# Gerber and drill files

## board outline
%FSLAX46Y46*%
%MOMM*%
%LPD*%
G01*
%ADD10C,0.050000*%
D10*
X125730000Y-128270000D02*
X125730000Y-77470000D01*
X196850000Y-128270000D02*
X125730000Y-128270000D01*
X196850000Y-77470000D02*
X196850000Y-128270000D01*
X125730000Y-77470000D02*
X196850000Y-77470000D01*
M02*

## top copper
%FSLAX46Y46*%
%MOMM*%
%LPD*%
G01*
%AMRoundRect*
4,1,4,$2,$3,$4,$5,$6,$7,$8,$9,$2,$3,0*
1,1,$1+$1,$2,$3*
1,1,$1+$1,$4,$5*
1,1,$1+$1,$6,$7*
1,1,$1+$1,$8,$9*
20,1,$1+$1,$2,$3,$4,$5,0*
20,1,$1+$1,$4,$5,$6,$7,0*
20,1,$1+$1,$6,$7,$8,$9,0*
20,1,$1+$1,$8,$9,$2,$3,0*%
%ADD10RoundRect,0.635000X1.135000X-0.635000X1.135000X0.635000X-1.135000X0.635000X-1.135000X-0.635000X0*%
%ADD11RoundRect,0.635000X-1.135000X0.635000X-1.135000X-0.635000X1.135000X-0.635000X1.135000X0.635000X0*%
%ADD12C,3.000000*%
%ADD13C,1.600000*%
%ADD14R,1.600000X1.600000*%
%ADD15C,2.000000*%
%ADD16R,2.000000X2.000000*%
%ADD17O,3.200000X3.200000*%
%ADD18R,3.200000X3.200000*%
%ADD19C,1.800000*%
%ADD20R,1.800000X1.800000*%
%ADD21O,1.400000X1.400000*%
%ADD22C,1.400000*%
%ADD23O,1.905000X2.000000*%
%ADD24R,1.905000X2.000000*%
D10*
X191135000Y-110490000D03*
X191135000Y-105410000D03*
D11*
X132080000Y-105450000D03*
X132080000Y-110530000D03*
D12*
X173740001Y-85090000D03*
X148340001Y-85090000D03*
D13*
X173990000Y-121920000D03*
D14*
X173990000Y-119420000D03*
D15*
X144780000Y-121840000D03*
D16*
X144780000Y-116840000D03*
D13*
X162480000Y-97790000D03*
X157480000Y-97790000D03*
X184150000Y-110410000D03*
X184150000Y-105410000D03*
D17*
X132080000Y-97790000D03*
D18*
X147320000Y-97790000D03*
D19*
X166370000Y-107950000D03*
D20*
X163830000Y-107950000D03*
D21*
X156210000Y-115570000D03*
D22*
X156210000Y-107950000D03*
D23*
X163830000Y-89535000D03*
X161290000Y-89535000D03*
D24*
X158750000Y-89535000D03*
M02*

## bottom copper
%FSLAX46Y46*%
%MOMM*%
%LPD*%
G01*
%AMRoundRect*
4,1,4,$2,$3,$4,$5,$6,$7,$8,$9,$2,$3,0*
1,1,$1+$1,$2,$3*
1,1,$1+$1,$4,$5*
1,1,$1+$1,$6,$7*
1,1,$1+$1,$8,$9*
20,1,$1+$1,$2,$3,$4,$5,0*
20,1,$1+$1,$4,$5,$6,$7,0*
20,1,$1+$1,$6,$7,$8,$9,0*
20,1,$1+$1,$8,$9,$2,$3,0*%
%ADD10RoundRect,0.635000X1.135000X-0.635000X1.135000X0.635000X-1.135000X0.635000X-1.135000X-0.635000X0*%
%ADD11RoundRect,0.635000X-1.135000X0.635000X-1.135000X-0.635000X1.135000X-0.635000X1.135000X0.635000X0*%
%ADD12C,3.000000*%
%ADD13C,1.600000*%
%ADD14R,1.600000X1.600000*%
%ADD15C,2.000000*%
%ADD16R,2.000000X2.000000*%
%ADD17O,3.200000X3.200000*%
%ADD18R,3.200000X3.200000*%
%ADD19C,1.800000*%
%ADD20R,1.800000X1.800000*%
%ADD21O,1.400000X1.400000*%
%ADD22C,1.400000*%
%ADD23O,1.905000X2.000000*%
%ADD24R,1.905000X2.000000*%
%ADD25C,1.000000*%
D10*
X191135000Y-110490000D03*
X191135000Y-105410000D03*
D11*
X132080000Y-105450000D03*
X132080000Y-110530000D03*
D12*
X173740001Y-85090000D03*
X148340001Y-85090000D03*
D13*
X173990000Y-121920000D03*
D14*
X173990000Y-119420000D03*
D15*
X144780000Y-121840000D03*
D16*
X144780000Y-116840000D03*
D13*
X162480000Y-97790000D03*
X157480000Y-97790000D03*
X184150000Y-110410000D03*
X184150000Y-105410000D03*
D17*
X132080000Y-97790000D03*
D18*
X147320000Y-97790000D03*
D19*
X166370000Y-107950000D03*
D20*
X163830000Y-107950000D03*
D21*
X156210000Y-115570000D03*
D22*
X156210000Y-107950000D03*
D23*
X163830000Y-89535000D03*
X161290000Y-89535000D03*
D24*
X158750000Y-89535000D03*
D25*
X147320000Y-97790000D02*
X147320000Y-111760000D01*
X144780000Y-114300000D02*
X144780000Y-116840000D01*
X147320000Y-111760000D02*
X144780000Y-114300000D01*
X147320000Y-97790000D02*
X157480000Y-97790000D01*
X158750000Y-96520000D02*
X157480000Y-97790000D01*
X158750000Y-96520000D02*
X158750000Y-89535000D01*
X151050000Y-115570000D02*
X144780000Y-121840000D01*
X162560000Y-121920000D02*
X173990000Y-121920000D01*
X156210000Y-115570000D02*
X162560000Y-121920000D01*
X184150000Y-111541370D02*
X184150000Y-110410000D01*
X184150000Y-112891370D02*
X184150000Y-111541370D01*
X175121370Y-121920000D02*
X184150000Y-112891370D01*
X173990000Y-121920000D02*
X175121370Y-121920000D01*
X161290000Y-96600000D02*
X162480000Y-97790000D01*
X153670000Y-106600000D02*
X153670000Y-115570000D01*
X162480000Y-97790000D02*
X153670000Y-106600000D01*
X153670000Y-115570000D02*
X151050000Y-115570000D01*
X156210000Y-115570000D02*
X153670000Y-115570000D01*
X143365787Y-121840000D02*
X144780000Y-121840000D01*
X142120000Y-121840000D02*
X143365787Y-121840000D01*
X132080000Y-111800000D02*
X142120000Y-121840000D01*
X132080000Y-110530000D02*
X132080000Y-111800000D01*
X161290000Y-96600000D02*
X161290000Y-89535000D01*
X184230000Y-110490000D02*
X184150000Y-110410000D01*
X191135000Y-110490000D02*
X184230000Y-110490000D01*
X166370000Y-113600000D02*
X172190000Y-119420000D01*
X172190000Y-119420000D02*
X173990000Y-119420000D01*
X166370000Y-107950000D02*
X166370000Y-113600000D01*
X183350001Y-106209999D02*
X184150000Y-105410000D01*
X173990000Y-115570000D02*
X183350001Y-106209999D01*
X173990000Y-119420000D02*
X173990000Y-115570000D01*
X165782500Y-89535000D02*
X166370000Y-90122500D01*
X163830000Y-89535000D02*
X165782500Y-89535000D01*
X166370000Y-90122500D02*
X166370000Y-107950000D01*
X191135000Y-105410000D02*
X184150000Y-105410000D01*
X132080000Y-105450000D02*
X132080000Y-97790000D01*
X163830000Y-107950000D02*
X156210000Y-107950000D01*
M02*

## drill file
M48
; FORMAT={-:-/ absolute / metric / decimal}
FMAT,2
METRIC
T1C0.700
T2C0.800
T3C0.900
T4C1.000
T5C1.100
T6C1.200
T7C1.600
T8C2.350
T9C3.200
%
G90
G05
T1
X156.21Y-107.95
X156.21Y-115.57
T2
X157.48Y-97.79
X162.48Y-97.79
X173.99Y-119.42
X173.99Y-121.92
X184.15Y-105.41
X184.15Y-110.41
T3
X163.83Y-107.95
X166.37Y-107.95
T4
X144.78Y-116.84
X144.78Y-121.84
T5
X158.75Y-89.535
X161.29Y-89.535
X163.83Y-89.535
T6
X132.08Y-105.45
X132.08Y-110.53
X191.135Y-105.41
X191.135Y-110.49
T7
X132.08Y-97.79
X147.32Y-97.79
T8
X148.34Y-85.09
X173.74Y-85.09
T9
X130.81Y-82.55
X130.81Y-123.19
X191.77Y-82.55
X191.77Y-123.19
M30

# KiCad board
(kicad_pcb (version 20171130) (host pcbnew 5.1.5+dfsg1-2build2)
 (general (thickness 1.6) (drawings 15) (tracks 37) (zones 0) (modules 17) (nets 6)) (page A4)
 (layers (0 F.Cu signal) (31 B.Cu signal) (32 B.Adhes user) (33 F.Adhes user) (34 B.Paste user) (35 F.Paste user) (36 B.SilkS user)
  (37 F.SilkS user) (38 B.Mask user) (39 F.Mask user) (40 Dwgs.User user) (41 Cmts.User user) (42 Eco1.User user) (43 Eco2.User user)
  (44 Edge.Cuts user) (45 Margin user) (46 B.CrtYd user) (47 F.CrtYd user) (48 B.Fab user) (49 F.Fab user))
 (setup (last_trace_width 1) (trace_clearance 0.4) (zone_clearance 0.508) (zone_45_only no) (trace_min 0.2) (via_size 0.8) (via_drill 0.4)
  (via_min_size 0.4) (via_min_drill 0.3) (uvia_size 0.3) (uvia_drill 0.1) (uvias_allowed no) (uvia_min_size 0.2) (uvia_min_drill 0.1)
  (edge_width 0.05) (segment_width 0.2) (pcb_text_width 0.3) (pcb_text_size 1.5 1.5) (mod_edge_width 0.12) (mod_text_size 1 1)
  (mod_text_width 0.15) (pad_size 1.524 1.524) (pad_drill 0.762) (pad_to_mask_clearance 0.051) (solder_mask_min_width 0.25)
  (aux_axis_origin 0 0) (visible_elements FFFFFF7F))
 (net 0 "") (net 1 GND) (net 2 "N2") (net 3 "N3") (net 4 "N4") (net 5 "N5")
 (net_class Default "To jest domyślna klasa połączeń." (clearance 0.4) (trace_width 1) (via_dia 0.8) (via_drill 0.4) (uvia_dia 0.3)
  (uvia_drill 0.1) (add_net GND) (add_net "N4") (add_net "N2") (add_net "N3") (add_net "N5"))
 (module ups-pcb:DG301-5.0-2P (layer F.Cu) (at 191.135 107.99 90)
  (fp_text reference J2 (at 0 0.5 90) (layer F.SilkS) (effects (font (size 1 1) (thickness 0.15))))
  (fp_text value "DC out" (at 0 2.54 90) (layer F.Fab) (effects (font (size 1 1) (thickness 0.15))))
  (pad 1 thru_hole roundrect (at -2.5 0 90) (size 2.54 3.54) (drill 1.2) (layers *.Cu *.Mask) (roundrect_rratio 0.25) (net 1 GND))
  (pad 2 thru_hole roundrect (at 2.58 0 90) (size 2.54 3.54) (drill 1.2) (layers *.Cu *.Mask) (roundrect_rratio 0.25) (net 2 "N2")))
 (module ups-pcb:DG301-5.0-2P (layer F.Cu) (at 132.08 107.95 270)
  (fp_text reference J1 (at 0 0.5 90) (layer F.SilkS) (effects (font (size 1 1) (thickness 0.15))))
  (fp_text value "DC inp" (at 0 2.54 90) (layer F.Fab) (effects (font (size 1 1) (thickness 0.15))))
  (pad 1 thru_hole roundrect (at -2.5 0 270) (size 2.54 3.54) (drill 1.2) (layers *.Cu *.Mask) (roundrect_rratio 0.25) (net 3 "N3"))
  (pad 2 thru_hole roundrect (at 2.58 0 270) (size 2.54 3.54) (drill 1.2) (layers *.Cu *.Mask) (roundrect_rratio 0.25) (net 1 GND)))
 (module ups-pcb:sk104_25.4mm (layer F.Cu) (at 161.040001 85.09)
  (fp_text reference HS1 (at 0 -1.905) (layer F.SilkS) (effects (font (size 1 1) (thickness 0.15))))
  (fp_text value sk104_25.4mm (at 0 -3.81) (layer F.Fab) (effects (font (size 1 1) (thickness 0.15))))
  (pad "" np_thru_hole circle (at 12.7 0) (size 3 3) (drill 2.35) (layers *.Cu *.Mask))
  (pad "" np_thru_hole circle (at -12.7 0) (size 3 3) (drill 2.35) (layers *.Cu *.Mask)))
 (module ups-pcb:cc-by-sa (layer F.Cu) (at 159.385 121.92)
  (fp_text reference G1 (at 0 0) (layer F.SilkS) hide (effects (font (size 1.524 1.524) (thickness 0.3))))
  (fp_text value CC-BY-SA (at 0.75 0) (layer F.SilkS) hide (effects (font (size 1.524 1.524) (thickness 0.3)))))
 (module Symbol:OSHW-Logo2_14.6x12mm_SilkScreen (layer F.Cu) (at 186.055 93.98)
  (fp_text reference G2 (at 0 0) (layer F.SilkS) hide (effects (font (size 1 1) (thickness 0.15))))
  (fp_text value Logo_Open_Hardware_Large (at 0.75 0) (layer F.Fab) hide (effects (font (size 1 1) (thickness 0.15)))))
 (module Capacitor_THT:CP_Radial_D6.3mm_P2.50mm (layer F.Cu) (at 173.99 119.42 270)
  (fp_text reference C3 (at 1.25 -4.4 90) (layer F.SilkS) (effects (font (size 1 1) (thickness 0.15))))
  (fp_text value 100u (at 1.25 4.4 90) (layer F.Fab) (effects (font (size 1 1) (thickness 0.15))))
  (pad 2 thru_hole circle (at 2.5 0 270) (size 1.6 1.6) (drill 0.8) (layers *.Cu *.Mask) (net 1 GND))
  (pad 1 thru_hole rect (at 0 0 270) (size 1.6 1.6) (drill 0.8) (layers *.Cu *.Mask) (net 2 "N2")))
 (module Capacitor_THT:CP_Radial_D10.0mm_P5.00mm (layer F.Cu) (at 144.78 116.84 270)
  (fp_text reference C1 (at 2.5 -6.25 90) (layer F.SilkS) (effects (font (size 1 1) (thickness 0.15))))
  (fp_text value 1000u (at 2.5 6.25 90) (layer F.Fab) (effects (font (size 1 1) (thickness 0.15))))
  (pad 2 thru_hole circle (at 5 0 270) (size 2 2) (drill 1) (layers *.Cu *.Mask) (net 1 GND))
  (pad 1 thru_hole rect (at 0 0 270) (size 2 2) (drill 1) (layers *.Cu *.Mask) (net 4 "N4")))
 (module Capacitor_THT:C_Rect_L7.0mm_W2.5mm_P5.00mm (layer F.Cu) (at 157.48 97.79)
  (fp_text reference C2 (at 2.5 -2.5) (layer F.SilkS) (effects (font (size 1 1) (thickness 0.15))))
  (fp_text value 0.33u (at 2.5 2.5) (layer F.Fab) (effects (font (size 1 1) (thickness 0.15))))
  (pad 2 thru_hole circle (at 5 0) (size 1.6 1.6) (drill 0.8) (layers *.Cu *.Mask) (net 1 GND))
  (pad 1 thru_hole circle (at 0 0) (size 1.6 1.6) (drill 0.8) (layers *.Cu *.Mask) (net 4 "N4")))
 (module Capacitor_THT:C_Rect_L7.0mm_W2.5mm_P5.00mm (layer F.Cu) (at 184.15 105.41 270)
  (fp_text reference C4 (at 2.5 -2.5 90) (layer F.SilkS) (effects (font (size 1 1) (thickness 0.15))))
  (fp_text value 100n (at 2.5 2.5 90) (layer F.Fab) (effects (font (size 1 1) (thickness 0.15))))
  (pad 2 thru_hole circle (at 5 0 270) (size 1.6 1.6) (drill 0.8) (layers *.Cu *.Mask) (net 1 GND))
  (pad 1 thru_hole circle (at 0 0 270) (size 1.6 1.6) (drill 0.8) (layers *.Cu *.Mask) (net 2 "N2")))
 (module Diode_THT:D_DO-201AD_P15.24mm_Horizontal (layer F.Cu) (at 147.32 97.79 180)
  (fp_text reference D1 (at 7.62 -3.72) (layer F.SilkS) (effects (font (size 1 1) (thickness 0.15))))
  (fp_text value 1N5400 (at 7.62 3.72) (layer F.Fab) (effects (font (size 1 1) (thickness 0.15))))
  (pad 2 thru_hole oval (at 15.24 0 180) (size 3.2 3.2) (drill 1.6) (layers *.Cu *.Mask) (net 3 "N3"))
  (pad 1 thru_hole rect (at 0 0 180) (size 3.2 3.2) (drill 1.6) (layers *.Cu *.Mask) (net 4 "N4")))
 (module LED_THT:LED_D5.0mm (layer F.Cu) (at 163.83 107.95)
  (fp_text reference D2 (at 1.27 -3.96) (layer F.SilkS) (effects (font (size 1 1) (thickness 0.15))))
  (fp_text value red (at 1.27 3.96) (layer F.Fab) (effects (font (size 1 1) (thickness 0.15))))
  (pad 2 thru_hole circle (at 2.54 0) (size 1.8 1.8) (drill 0.9) (layers *.Cu *.Mask) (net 2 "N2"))
  (pad 1 thru_hole rect (at 0 0) (size 1.8 1.8) (drill 0.9) (layers *.Cu *.Mask) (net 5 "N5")))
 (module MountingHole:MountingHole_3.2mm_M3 (layer F.Cu) (at 130.81 82.55)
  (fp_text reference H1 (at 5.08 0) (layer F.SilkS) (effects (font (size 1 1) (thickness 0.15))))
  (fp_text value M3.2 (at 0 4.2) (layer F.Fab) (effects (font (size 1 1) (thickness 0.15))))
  (pad 1 np_thru_hole circle (at 0 0) (size 3.2 3.2) (drill 3.2) (layers *.Cu *.Mask)))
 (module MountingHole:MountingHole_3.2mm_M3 (layer F.Cu) (at 191.77 82.55)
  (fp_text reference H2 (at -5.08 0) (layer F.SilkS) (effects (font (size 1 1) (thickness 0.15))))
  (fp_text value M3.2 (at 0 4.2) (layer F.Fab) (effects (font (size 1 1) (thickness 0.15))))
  (pad 1 np_thru_hole circle (at 0 0) (size 3.2 3.2) (drill 3.2) (layers *.Cu *.Mask)))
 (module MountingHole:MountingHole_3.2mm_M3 (layer F.Cu) (at 191.77 123.19)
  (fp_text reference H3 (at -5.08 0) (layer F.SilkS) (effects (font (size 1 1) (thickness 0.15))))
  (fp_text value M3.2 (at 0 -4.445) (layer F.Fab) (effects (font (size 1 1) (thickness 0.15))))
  (pad 1 np_thru_hole circle (at 0 0) (size 3.2 3.2) (drill 3.2) (layers *.Cu *.Mask)))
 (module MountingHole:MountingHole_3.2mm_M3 (layer F.Cu) (at 130.81 123.19)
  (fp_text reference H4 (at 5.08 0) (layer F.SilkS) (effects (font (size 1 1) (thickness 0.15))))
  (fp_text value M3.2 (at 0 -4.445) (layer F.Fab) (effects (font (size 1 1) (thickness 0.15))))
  (pad 1 np_thru_hole circle (at 0 0) (size 3.2 3.2) (drill 3.2) (layers *.Cu *.Mask)))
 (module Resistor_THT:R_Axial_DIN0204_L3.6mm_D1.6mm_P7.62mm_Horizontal (layer F.Cu) (at 156.21 107.95 270)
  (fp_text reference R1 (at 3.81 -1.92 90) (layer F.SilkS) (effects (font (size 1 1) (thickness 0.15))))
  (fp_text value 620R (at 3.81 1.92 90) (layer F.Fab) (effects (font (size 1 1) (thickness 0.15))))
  (pad 2 thru_hole oval (at 7.62 0 270) (size 1.4 1.4) (drill 0.7) (layers *.Cu *.Mask) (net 1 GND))
  (pad 1 thru_hole circle (at 0 0 270) (size 1.4 1.4) (drill 0.7) (layers *.Cu *.Mask) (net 5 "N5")))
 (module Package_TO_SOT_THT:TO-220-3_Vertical (layer F.Cu) (at 158.75 89.535)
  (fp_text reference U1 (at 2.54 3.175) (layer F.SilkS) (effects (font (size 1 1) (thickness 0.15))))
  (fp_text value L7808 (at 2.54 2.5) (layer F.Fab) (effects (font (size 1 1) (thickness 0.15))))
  (pad 3 thru_hole oval (at 5.08 0) (size 1.905 2) (drill 1.1) (layers *.Cu *.Mask) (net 2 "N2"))
  (pad 2 thru_hole oval (at 2.54 0) (size 1.905 2) (drill 1.1) (layers *.Cu *.Mask) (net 1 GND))
  (pad 1 thru_hole rect (at 0 0) (size 1.905 2) (drill 1.1) (layers *.Cu *.Mask) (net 4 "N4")))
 (gr_line (start 125.73 128.27) (end 125.73 77.47) (layer Edge.Cuts) (width 0.05))
 (gr_line (start 196.85 128.27) (end 125.73 128.27) (layer Edge.Cuts) (width 0.05))
 (gr_line (start 196.85 77.47) (end 196.85 128.27) (layer Edge.Cuts) (width 0.05))
 (gr_line (start 125.73 77.47) (end 196.85 77.47) (layer Edge.Cuts) (width 0.05))
 (segment (start 147.32 97.79) (end 147.32 111.76) (width 1) (layer B.Cu) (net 4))
 (segment (start 144.78 114.3) (end 144.78 116.84) (width 1) (layer B.Cu) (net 4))
 (segment (start 147.32 111.76) (end 144.78 114.3) (width 1) (layer B.Cu) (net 4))
 (segment (start 147.32 97.79) (end 157.48 97.79) (width 1) (layer B.Cu) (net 4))
 (segment (start 158.75 96.52) (end 157.48 97.79) (width 1) (layer B.Cu) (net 4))
 (segment (start 158.75 96.52) (end 158.75 89.535) (width 1) (layer B.Cu) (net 4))
 (segment (start 151.05 115.57) (end 144.78 121.84) (width 1) (layer B.Cu) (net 1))
 (segment (start 162.56 121.92) (end 173.99 121.92) (width 1) (layer B.Cu) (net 1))
 (segment (start 156.21 115.57) (end 162.56 121.92) (width 1) (layer B.Cu) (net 1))
 (segment (start 184.15 111.54137) (end 184.15 110.41) (width 1) (layer B.Cu) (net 1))
 (segment (start 184.15 112.89137) (end 184.15 111.54137) (width 1) (layer B.Cu) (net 1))
 (segment (start 175.12137 121.92) (end 184.15 112.89137) (width 1) (layer B.Cu) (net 1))
 (segment (start 173.99 121.92) (end 175.12137 121.92) (width 1) (layer B.Cu) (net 1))
 (segment (start 161.29 96.6) (end 162.48 97.79) (width 1) (layer B.Cu) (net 1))
 (segment (start 153.67 106.6) (end 153.67 115.57) (width 1) (layer B.Cu) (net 1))
 (segment (start 162.48 97.79) (end 153.67 106.6) (width 1) (layer B.Cu) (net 1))
 (segment (start 153.67 115.57) (end 151.05 115.57) (width 1) (layer B.Cu) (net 1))
 (segment (start 156.21 115.57) (end 153.67 115.57) (width 1) (layer B.Cu) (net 1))
 (segment (start 143.365787 121.84) (end 144.78 121.84) (width 1) (layer B.Cu) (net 1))
 (segment (start 142.12 121.84) (end 143.365787 121.84) (width 1) (layer B.Cu) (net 1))
 (segment (start 132.08 111.8) (end 142.12 121.84) (width 1) (layer B.Cu) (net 1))
 (segment (start 132.08 110.53) (end 132.08 111.8) (width 1) (layer B.Cu) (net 1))
 (segment (start 161.29 96.6) (end 161.29 89.535) (width 1) (layer B.Cu) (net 1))
 (segment (start 184.23 110.49) (end 184.15 110.41) (width 1) (layer B.Cu) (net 1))
 (segment (start 191.135 110.49) (end 184.23 110.49) (width 1) (layer B.Cu) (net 1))
 (segment (start 166.37 113.6) (end 172.19 119.42) (width 1) (layer B.Cu) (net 2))
 (segment (start 172.19 119.42) (end 173.99 119.42) (width 1) (layer B.Cu) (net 2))
 (segment (start 166.37 107.95) (end 166.37 113.6) (width 1) (layer B.Cu) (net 2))
 (segment (start 183.350001 106.209999) (end 184.15 105.41) (width 1) (layer B.Cu) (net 2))
 (segment (start 173.99 115.57) (end 183.350001 106.209999) (width 1) (layer B.Cu) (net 2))
 (segment (start 173.99 119.42) (end 173.99 115.57) (width 1) (layer B.Cu) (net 2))
 (segment (start 165.7825 89.535) (end 166.37 90.1225) (width 1) (layer B.Cu) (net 2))
 (segment (start 163.83 89.535) (end 165.7825 89.535) (width 1) (layer B.Cu) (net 2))
 (segment (start 166.37 90.1225) (end 166.37 107.95) (width 1) (layer B.Cu) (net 2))
 (segment (start 191.135 105.41) (end 184.15 105.41) (width 1) (layer B.Cu) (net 2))
 (segment (start 132.08 105.45) (end 132.08 97.79) (width 1) (layer B.Cu) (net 3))
 (segment (start 163.83 107.95) (end 156.21 107.95) (width 1) (layer B.Cu) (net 5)))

